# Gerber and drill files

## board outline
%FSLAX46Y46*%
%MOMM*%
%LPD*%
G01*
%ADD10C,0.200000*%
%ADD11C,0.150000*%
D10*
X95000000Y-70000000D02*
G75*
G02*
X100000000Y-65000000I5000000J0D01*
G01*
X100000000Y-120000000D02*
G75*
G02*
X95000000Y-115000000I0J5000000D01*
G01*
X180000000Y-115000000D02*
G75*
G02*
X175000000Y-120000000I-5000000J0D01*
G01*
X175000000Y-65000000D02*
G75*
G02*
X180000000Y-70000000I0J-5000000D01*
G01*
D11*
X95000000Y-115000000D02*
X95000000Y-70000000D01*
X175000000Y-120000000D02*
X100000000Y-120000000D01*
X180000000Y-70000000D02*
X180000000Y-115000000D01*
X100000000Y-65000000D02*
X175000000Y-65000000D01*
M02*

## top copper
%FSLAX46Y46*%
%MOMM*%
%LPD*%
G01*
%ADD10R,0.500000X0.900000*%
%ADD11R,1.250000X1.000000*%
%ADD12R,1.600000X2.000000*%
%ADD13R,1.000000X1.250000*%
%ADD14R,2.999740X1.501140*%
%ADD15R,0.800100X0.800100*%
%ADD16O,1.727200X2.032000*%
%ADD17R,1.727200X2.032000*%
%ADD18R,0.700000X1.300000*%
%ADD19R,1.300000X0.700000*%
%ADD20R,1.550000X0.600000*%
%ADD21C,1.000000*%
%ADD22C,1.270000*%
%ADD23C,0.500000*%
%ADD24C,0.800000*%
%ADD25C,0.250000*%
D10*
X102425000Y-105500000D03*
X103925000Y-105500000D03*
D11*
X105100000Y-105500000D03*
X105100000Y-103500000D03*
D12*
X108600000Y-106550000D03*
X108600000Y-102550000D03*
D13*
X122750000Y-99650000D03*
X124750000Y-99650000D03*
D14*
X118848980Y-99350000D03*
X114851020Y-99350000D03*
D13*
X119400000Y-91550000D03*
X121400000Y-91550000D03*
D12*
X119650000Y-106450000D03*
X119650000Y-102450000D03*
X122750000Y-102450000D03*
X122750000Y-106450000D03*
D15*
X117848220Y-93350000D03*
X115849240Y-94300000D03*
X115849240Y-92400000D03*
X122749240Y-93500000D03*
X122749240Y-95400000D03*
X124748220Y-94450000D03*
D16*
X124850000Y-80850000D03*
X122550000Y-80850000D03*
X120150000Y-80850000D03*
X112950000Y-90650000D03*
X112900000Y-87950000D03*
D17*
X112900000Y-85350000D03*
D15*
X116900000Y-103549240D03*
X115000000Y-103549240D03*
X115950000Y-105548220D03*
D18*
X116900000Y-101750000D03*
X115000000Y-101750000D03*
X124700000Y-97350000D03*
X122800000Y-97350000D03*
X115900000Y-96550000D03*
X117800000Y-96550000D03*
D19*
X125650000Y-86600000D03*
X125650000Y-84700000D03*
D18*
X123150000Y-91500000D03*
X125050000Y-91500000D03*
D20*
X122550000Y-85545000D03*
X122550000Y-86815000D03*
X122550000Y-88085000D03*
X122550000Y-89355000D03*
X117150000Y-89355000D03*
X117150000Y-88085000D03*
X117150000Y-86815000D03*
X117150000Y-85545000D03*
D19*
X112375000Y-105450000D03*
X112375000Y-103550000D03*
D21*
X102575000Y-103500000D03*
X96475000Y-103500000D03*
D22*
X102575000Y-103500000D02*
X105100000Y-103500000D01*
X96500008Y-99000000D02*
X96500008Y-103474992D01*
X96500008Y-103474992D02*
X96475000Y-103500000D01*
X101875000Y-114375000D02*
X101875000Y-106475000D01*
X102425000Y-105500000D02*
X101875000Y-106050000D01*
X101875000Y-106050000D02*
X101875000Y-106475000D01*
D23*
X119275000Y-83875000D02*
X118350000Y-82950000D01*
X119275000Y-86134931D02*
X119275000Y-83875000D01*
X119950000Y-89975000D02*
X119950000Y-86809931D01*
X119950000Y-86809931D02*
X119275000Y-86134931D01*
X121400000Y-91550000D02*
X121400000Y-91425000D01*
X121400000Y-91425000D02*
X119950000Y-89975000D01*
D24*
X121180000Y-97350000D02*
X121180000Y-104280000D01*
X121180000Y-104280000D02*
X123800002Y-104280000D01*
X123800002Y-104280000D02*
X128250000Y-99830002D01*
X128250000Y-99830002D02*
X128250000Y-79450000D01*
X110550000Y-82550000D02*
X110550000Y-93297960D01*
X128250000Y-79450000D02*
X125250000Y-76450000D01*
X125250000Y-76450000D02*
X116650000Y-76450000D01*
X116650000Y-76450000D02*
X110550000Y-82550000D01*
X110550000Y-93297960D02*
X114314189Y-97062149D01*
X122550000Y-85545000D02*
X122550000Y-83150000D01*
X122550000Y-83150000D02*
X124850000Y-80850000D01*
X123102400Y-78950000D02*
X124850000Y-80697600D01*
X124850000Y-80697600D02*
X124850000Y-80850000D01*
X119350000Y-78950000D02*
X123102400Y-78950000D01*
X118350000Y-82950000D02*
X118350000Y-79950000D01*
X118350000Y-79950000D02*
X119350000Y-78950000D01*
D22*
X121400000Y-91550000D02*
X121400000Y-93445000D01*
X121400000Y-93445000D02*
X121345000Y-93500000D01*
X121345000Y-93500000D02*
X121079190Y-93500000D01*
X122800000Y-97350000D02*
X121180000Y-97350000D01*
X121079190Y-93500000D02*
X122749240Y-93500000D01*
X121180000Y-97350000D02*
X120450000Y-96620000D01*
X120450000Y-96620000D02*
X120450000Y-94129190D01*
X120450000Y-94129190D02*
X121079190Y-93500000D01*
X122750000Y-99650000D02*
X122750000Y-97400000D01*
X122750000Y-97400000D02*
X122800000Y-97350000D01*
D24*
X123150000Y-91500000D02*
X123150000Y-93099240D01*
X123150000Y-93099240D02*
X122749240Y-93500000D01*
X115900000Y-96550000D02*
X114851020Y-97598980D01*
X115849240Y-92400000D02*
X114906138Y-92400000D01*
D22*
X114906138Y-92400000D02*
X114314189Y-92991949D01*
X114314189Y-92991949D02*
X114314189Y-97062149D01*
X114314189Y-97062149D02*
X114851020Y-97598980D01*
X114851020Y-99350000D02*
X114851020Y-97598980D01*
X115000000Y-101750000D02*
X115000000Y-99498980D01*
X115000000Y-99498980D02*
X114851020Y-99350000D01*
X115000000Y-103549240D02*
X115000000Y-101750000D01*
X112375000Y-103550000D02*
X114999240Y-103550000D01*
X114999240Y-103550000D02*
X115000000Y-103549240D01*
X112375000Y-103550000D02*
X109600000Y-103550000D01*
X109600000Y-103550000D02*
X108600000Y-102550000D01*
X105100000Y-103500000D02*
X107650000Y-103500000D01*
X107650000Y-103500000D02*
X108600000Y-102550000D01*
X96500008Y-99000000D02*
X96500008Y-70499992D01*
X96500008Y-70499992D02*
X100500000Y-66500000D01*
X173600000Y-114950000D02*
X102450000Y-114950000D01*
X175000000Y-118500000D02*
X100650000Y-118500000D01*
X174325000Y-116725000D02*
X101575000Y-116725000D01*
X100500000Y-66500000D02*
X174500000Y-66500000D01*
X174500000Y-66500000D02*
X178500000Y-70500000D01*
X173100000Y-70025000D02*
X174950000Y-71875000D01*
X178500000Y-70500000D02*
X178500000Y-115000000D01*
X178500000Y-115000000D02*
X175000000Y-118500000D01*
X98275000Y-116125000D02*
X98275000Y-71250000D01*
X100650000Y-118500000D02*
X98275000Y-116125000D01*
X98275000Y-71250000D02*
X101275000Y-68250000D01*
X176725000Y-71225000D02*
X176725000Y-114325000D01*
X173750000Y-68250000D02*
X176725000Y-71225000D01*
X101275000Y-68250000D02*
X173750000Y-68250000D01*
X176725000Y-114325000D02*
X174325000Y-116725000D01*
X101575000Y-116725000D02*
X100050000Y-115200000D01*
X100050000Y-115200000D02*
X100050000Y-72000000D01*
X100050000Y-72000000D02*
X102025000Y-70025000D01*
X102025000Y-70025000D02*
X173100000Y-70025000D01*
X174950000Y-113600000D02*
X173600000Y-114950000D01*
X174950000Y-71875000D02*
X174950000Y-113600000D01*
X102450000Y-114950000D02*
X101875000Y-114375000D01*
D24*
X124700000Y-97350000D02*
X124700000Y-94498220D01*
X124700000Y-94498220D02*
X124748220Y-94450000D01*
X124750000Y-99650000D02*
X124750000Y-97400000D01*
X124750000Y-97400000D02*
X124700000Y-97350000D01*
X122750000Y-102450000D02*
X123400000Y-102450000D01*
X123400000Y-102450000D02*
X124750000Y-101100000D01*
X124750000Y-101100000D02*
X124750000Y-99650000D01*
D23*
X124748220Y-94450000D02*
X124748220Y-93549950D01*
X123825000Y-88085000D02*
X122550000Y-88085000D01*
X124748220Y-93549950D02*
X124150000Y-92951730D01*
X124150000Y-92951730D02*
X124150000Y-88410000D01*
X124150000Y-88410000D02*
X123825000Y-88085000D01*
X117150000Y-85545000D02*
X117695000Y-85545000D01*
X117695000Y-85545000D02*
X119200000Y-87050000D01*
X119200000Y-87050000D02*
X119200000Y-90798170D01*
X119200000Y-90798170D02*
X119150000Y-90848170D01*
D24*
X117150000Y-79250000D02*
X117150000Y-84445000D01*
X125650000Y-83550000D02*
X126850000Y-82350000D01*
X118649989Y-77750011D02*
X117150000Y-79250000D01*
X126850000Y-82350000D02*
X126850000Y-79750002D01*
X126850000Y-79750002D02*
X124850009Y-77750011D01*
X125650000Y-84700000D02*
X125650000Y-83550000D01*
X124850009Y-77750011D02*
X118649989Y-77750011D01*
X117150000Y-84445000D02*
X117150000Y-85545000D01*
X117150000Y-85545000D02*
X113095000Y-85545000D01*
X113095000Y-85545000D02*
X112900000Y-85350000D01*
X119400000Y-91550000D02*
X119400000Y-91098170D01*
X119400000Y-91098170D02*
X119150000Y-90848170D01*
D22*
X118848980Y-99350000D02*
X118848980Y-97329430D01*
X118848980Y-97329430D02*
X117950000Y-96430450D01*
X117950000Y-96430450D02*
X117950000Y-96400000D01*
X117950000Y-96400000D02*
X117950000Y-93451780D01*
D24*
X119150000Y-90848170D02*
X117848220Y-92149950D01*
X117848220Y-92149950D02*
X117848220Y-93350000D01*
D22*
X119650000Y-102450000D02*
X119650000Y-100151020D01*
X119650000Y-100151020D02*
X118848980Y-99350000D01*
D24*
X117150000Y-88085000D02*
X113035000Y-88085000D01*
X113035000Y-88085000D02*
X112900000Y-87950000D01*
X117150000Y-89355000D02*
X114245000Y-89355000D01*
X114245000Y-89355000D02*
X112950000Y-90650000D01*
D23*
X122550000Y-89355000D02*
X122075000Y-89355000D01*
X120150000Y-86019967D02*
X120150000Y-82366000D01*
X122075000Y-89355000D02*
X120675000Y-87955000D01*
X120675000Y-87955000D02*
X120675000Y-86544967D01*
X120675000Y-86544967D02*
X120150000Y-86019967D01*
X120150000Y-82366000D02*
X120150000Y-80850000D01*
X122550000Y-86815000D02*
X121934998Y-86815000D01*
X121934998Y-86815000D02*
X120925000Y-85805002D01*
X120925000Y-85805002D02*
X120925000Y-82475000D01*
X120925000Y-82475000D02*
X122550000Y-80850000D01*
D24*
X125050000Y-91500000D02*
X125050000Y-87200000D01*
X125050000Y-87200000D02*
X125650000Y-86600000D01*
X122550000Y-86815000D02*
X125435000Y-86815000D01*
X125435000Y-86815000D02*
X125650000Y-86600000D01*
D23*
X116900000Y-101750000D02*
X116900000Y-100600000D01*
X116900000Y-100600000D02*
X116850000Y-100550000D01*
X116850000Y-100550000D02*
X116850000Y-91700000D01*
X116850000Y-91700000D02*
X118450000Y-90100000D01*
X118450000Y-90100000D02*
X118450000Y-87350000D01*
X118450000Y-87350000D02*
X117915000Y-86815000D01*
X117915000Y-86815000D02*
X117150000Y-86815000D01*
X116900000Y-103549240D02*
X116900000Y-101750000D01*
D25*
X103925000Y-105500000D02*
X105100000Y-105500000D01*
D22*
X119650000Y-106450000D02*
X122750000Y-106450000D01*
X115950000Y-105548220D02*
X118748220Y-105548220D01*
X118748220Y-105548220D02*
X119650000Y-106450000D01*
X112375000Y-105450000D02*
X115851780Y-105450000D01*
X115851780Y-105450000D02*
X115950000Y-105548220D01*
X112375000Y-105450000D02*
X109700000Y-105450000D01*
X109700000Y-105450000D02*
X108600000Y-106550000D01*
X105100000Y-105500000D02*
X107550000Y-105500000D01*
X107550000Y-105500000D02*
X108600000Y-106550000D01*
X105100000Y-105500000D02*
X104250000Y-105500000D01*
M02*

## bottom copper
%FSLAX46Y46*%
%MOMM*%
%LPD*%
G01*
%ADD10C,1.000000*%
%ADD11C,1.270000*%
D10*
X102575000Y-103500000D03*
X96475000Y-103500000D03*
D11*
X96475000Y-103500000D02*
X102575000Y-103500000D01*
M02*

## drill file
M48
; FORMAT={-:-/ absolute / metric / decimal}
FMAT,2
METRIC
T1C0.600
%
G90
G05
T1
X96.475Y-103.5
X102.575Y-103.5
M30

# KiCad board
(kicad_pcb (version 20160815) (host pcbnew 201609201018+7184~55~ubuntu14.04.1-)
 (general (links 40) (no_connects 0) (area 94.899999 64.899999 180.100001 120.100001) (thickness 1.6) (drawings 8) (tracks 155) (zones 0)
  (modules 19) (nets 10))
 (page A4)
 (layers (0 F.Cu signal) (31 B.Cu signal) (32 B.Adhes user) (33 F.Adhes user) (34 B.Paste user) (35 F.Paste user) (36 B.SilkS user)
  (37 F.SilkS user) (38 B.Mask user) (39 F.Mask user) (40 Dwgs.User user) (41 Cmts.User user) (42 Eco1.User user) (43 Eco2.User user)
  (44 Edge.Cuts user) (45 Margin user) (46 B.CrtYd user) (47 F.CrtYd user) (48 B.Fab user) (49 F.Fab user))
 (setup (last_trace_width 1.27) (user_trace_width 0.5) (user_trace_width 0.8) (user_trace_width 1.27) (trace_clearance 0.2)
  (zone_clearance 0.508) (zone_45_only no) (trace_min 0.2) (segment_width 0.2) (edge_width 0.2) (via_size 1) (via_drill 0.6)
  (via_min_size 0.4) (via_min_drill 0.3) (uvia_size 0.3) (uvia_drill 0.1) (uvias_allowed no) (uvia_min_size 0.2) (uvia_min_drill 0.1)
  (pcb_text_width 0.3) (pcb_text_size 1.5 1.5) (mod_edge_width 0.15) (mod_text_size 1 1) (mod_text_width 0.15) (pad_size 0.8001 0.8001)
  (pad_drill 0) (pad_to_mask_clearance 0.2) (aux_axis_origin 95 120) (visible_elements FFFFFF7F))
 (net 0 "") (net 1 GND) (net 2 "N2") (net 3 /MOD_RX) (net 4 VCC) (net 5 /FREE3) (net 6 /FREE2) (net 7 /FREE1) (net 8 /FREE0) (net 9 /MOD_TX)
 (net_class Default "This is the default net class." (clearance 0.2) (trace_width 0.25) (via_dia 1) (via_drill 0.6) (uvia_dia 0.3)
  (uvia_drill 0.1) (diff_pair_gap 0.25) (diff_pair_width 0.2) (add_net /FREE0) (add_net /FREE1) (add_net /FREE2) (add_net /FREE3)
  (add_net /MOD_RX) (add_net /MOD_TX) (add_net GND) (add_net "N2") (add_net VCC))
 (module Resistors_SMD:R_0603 (layer F.Cu) (at 103.175 105.5 180)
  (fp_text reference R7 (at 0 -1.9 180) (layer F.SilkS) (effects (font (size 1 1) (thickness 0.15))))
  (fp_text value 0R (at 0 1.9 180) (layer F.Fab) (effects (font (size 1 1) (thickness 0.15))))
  (pad 2 smd rect (at 0.75 0 180) (size 0.5 0.9) (layers F.Cu F.Paste F.Mask) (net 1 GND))
  (pad 1 smd rect (at -0.75 0 180) (size 0.5 0.9) (layers F.Cu F.Paste F.Mask) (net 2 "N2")))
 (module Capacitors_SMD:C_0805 (layer F.Cu) (at 105.1 104.5 90)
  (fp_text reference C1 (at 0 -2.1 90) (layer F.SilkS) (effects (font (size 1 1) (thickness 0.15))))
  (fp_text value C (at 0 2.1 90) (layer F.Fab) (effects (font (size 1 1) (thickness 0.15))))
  (pad 1 smd rect (at -1 0 90) (size 1 1.25) (layers F.Cu F.Paste F.Mask) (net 2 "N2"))
  (pad 2 smd rect (at 1 0 90) (size 1 1.25) (layers F.Cu F.Paste F.Mask) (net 1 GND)))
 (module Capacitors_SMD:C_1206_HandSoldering (layer F.Cu) (at 108.6 104.55 90)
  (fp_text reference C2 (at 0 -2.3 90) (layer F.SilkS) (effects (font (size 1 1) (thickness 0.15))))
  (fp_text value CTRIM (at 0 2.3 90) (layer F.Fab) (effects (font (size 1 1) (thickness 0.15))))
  (pad 1 smd rect (at -2 0 90) (size 2 1.6) (layers F.Cu F.Paste F.Mask) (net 2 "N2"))
  (pad 2 smd rect (at 2 0 90) (size 2 1.6) (layers F.Cu F.Paste F.Mask) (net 1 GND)))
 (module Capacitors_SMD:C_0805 (layer F.Cu) (at 123.75 99.65 180)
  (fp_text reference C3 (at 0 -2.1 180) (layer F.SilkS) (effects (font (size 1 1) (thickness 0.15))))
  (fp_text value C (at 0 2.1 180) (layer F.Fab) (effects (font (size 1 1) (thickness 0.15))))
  (pad 2 smd rect (at 1 0 180) (size 1 1.25) (layers F.Cu F.Paste F.Mask) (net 1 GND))
  (pad 1 smd rect (at -1 0 180) (size 1 1.25) (layers F.Cu F.Paste F.Mask) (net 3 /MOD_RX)))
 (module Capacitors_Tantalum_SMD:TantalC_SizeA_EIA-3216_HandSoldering (layer F.Cu) (at 116.85 99.35 180)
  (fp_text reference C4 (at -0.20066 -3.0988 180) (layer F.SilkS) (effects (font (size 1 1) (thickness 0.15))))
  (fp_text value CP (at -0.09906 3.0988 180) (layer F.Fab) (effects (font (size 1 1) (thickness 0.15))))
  (pad 1 smd rect (at -1.99898 0 180) (size 2.99974 1.50114) (layers F.Cu F.Paste F.Mask) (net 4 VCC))
  (pad 2 smd rect (at 1.99898 0 180) (size 2.99974 1.50114) (layers F.Cu F.Paste F.Mask) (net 1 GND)))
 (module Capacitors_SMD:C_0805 (layer F.Cu) (at 120.4 91.55)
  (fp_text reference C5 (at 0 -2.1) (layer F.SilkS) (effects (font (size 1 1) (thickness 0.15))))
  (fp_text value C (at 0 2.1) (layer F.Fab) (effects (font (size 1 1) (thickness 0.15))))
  (pad 1 smd rect (at -1 0) (size 1 1.25) (layers F.Cu F.Paste F.Mask) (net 4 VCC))
  (pad 2 smd rect (at 1 0) (size 1 1.25) (layers F.Cu F.Paste F.Mask) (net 1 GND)))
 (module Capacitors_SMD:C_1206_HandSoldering (layer F.Cu) (at 119.65 104.45 270)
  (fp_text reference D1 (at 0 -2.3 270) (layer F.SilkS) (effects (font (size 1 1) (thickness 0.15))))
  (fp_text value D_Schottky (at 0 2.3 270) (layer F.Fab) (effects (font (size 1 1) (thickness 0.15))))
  (pad 2 smd rect (at 2 0 270) (size 2 1.6) (layers F.Cu F.Paste F.Mask) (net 2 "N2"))
  (pad 1 smd rect (at -2 0 270) (size 2 1.6) (layers F.Cu F.Paste F.Mask) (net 4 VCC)))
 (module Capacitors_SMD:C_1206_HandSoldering (layer F.Cu) (at 122.75 104.45 270)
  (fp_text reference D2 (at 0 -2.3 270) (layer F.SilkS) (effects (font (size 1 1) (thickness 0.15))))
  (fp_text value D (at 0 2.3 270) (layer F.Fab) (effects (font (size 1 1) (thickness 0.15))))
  (pad 1 smd rect (at -2 0 270) (size 2 1.6) (layers F.Cu F.Paste F.Mask) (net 3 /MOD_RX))
  (pad 2 smd rect (at 2 0 270) (size 2 1.6) (layers F.Cu F.Paste F.Mask) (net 2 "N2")))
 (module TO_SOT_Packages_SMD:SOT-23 (layer F.Cu) (at 116.85 93.35 270)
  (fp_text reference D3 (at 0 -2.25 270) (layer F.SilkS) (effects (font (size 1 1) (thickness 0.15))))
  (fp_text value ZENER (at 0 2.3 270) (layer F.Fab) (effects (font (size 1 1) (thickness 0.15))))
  (pad 1 smd rect (at 0 -0.99822 270) (size 0.8001 0.8001) (layers F.Cu F.Paste F.Mask) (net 4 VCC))
  (pad 3 smd rect (at 0.95 1.00076 270) (size 0.8001 0.8001) (layers F.Cu F.Paste F.Mask))
  (pad 2 smd rect (at -0.95 1.00076 270) (size 0.8001 0.8001) (layers F.Cu F.Paste F.Mask) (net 1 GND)))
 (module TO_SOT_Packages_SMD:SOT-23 (layer F.Cu) (at 123.75 94.45 270)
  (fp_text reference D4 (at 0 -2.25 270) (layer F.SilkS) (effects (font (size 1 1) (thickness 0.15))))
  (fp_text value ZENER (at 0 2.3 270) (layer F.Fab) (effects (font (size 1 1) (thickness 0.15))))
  (pad 2 smd rect (at -0.95 1.00076 270) (size 0.8001 0.8001) (layers F.Cu F.Paste F.Mask) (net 1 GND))
  (pad 3 smd rect (at 0.95 1.00076 270) (size 0.8001 0.8001) (layers F.Cu F.Paste F.Mask))
  (pad 1 smd rect (at 0 -0.99822 270) (size 0.8001 0.8001) (layers F.Cu F.Paste F.Mask) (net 3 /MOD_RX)))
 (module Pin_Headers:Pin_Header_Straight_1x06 (layer F.Cu) (at 114.17 80.65 90)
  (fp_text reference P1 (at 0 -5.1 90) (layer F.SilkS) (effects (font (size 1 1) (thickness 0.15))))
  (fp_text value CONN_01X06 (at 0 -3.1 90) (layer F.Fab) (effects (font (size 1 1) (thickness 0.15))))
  (pad 6 smd oval (at -0.2 10.68 90) (size 2.032 1.7272) (layers F.Cu F.Paste F.Mask) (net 1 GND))
  (pad 5 smd oval (at -0.2 8.38 90) (size 2.032 1.7272) (layers F.Cu F.Paste F.Mask) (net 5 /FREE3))
  (pad 4 smd oval (at -0.2 5.98 90) (size 2.032 1.7272) (layers F.Cu F.Paste F.Mask) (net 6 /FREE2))
  (pad 3 smd oval (at -10 -1.22 90) (size 2.032 1.7272) (layers F.Cu F.Paste F.Mask) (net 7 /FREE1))
  (pad 2 smd oval (at -7.3 -1.27 90) (size 2.032 1.7272) (layers F.Cu F.Paste F.Mask) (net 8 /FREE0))
  (pad 1 smd rect (at -4.7 -1.27 90) (size 2.032 1.7272) (layers F.Cu F.Paste F.Mask) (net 4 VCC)))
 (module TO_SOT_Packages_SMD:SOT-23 (layer F.Cu) (at 115.95 104.55 180)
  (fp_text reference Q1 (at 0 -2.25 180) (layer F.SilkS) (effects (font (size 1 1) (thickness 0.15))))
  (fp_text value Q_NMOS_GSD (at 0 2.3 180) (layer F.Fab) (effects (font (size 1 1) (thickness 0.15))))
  (pad 1 smd rect (at -0.95 1.00076 180) (size 0.8001 0.8001) (layers F.Cu F.Paste F.Mask) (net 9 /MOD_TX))
  (pad 2 smd rect (at 0.95 1.00076 180) (size 0.8001 0.8001) (layers F.Cu F.Paste F.Mask) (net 1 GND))
  (pad 3 smd rect (at 0 -0.99822 180) (size 0.8001 0.8001) (layers F.Cu F.Paste F.Mask) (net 2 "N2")))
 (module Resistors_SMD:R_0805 (layer F.Cu) (at 115.95 101.75 180)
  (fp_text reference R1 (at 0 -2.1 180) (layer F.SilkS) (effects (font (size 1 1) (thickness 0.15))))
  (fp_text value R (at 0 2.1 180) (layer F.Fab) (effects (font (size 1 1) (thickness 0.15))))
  (pad 1 smd rect (at -0.95 0 180) (size 0.7 1.3) (layers F.Cu F.Paste F.Mask) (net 9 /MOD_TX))
  (pad 2 smd rect (at 0.95 0 180) (size 0.7 1.3) (layers F.Cu F.Paste F.Mask) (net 1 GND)))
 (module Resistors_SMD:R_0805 (layer F.Cu) (at 123.75 97.35 180)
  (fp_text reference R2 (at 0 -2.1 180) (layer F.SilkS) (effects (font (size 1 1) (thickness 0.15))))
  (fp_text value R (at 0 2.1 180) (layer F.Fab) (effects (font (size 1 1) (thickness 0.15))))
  (pad 1 smd rect (at -0.95 0 180) (size 0.7 1.3) (layers F.Cu F.Paste F.Mask) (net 3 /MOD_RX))
  (pad 2 smd rect (at 0.95 0 180) (size 0.7 1.3) (layers F.Cu F.Paste F.Mask) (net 1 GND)))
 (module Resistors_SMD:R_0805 (layer F.Cu) (at 116.85 96.55 180)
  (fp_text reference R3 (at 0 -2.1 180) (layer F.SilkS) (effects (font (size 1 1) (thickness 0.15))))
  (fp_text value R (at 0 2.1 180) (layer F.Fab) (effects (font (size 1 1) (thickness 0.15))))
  (pad 2 smd rect (at 0.95 0 180) (size 0.7 1.3) (layers F.Cu F.Paste F.Mask) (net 1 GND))
  (pad 1 smd rect (at -0.95 0 180) (size 0.7 1.3) (layers F.Cu F.Paste F.Mask) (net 4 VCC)))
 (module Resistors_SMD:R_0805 (layer F.Cu) (at 125.65 85.65 270)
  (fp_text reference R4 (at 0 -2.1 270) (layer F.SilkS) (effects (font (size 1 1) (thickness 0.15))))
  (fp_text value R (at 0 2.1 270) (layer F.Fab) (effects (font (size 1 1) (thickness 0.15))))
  (pad 2 smd rect (at 0.95 0 270) (size 0.7 1.3) (layers F.Cu F.Paste F.Mask) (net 5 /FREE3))
  (pad 1 smd rect (at -0.95 0 270) (size 0.7 1.3) (layers F.Cu F.Paste F.Mask) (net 4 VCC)))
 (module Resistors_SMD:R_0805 (layer F.Cu) (at 124.1 91.5 180)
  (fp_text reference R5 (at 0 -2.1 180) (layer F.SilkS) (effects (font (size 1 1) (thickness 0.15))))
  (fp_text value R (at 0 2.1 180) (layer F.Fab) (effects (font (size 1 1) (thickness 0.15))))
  (pad 2 smd rect (at 0.95 0 180) (size 0.7 1.3) (layers F.Cu F.Paste F.Mask) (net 1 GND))
  (pad 1 smd rect (at -0.95 0 180) (size 0.7 1.3) (layers F.Cu F.Paste F.Mask) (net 5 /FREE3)))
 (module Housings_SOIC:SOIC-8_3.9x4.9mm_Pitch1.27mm (layer F.Cu) (at 119.85 87.45)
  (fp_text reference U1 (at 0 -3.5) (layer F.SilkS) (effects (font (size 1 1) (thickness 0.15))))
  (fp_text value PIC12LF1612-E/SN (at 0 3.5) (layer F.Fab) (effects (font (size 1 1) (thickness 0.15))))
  (pad 8 smd rect (at 2.7 -1.905) (size 1.55 0.6) (layers F.Cu F.Paste F.Mask) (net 1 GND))
  (pad 7 smd rect (at 2.7 -0.635) (size 1.55 0.6) (layers F.Cu F.Paste F.Mask) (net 5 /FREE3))
  (pad 6 smd rect (at 2.7 0.635) (size 1.55 0.6) (layers F.Cu F.Paste F.Mask) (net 3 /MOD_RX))
  (pad 5 smd rect (at 2.7 1.905) (size 1.55 0.6) (layers F.Cu F.Paste F.Mask) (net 6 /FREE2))
  (pad 4 smd rect (at -2.7 1.905) (size 1.55 0.6) (layers F.Cu F.Paste F.Mask) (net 7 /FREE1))
  (pad 3 smd rect (at -2.7 0.635) (size 1.55 0.6) (layers F.Cu F.Paste F.Mask) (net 8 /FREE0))
  (pad 2 smd rect (at -2.7 -0.635) (size 1.55 0.6) (layers F.Cu F.Paste F.Mask) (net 9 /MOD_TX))
  (pad 1 smd rect (at -2.7 -1.905) (size 1.55 0.6) (layers F.Cu F.Paste F.Mask) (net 4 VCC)))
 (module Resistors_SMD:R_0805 (layer F.Cu) (at 112.375 104.5 90)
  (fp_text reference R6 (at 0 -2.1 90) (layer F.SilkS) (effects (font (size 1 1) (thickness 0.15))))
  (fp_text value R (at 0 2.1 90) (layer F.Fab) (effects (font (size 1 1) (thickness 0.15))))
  (pad 1 smd rect (at -0.95 0 90) (size 0.7 1.3) (layers F.Cu F.Paste F.Mask) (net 2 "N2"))
  (pad 2 smd rect (at 0.95 0 90) (size 0.7 1.3) (layers F.Cu F.Paste F.Mask) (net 1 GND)))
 (gr_arc (start 100 70) (end 95 70) (angle 90) (layer Edge.Cuts) (width 0.2))
 (gr_arc (start 100 115) (end 100 120) (angle 90) (layer Edge.Cuts) (width 0.2))
 (gr_arc (start 175 115) (end 180 115) (angle 90) (layer Edge.Cuts) (width 0.2))
 (gr_arc (start 175 70) (end 175 65) (angle 90) (layer Edge.Cuts) (width 0.2))
 (gr_line (start 95 115) (end 95 70) (layer Edge.Cuts) (width 0.15))
 (gr_line (start 175 120) (end 100 120) (layer Edge.Cuts) (width 0.15))
 (gr_line (start 180 70) (end 180 115) (layer Edge.Cuts) (width 0.15))
 (gr_line (start 100 65) (end 175 65) (layer Edge.Cuts) (width 0.15))
 (segment (start 102.575 103.5) (end 105.1 103.5) (width 1.27) (layer F.Cu) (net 1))
 (segment (start 96.475 103.5) (end 102.575 103.5) (width 1.27) (layer B.Cu) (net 1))
 (via (at 102.575 103.5) (size 1) (drill 0.6) (layers F.Cu B.Cu) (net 1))
 (segment (start 96.500008 99) (end 96.500008 103.474992) (width 1.27) (layer F.Cu) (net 1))
 (segment (start 96.500008 103.474992) (end 96.475 103.5) (width 1.27) (layer F.Cu) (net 1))
 (via (at 96.475 103.5) (size 1) (drill 0.6) (layers F.Cu B.Cu) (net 1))
 (segment (start 101.875 114.375) (end 101.875 106.475) (width 1.27) (layer F.Cu) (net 1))
 (segment (start 102.425 105.5) (end 101.875 106.05) (width 1.27) (layer F.Cu) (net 1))
 (segment (start 101.875 106.05) (end 101.875 106.475) (width 1.27) (layer F.Cu) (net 1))
 (segment (start 119.275 83.875) (end 118.35 82.95) (width 0.5) (layer F.Cu) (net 1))
 (segment (start 119.275 86.134931) (end 119.275 83.875) (width 0.5) (layer F.Cu) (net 1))
 (segment (start 119.95 89.975) (end 119.95 86.809931) (width 0.5) (layer F.Cu) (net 1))
 (segment (start 119.95 86.809931) (end 119.275 86.134931) (width 0.5) (layer F.Cu) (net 1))
 (segment (start 121.4 91.55) (end 121.4 91.425) (width 0.5) (layer F.Cu) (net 1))
 (segment (start 121.4 91.425) (end 119.95 89.975) (width 0.5) (layer F.Cu) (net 1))
 (segment (start 121.18 97.35) (end 121.18 104.28) (width 0.8) (layer F.Cu) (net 1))
 (segment (start 121.18 104.28) (end 123.800002 104.28) (width 0.8) (layer F.Cu) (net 1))
 (segment (start 123.800002 104.28) (end 128.25 99.830002) (width 0.8) (layer F.Cu) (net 1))
 (segment (start 128.25 99.830002) (end 128.25 79.45) (width 0.8) (layer F.Cu) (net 1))
 (segment (start 110.55 82.55) (end 110.55 93.29796) (width 0.8) (layer F.Cu) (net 1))
 (segment (start 128.25 79.45) (end 125.25 76.45) (width 0.8) (layer F.Cu) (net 1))
 (segment (start 125.25 76.45) (end 116.65 76.45) (width 0.8) (layer F.Cu) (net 1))
 (segment (start 116.65 76.45) (end 110.55 82.55) (width 0.8) (layer F.Cu) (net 1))
 (segment (start 110.55 93.29796) (end 114.314189 97.062149) (width 0.8) (layer F.Cu) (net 1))
 (segment (start 122.55 85.545) (end 122.55 83.15) (width 0.8) (layer F.Cu) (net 1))
 (segment (start 122.55 83.15) (end 124.85 80.85) (width 0.8) (layer F.Cu) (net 1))
 (segment (start 123.1024 78.95) (end 124.85 80.6976) (width 0.8) (layer F.Cu) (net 1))
 (segment (start 124.85 80.6976) (end 124.85 80.85) (width 0.8) (layer F.Cu) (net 1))
 (segment (start 119.35 78.95) (end 123.1024 78.95) (width 0.8) (layer F.Cu) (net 1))
 (segment (start 118.35 82.95) (end 118.35 79.95) (width 0.8) (layer F.Cu) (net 1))
 (segment (start 118.35 79.95) (end 119.35 78.95) (width 0.8) (layer F.Cu) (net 1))
 (segment (start 121.4 91.55) (end 121.4 93.445) (width 1.27) (layer F.Cu) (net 1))
 (segment (start 121.4 93.445) (end 121.345 93.5) (width 1.27) (layer F.Cu) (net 1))
 (segment (start 121.345 93.5) (end 121.07919 93.5) (width 1.27) (layer F.Cu) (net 1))
 (segment (start 122.8 97.35) (end 121.18 97.35) (width 1.27) (layer F.Cu) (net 1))
 (segment (start 121.07919 93.5) (end 122.74924 93.5) (width 1.27) (layer F.Cu) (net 1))
 (segment (start 121.18 97.35) (end 120.45 96.62) (width 1.27) (layer F.Cu) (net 1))
 (segment (start 120.45 96.62) (end 120.45 94.12919) (width 1.27) (layer F.Cu) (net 1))
 (segment (start 120.45 94.12919) (end 121.07919 93.5) (width 1.27) (layer F.Cu) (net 1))
 (segment (start 122.75 99.65) (end 122.75 97.4) (width 1.27) (layer F.Cu) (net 1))
 (segment (start 122.75 97.4) (end 122.8 97.35) (width 1.27) (layer F.Cu) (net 1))
 (segment (start 123.15 91.5) (end 123.15 93.09924) (width 0.8) (layer F.Cu) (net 1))
 (segment (start 123.15 93.09924) (end 122.74924 93.5) (width 0.8) (layer F.Cu) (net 1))
 (segment (start 115.9 96.55) (end 114.85102 97.59898) (width 0.8) (layer F.Cu) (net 1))
 (segment (start 115.84924 92.4) (end 114.906138 92.4) (width 0.8) (layer F.Cu) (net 1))
 (segment (start 114.906138 92.4) (end 114.314189 92.991949) (width 1.27) (layer F.Cu) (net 1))
 (segment (start 114.314189 92.991949) (end 114.314189 97.062149) (width 1.27) (layer F.Cu) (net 1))
 (segment (start 114.314189 97.062149) (end 114.85102 97.59898) (width 1.27) (layer F.Cu) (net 1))
 (segment (start 114.85102 99.35) (end 114.85102 97.59898) (width 1.27) (layer F.Cu) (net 1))
 (segment (start 115 101.75) (end 115 99.49898) (width 1.27) (layer F.Cu) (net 1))
 (segment (start 115 99.49898) (end 114.85102 99.35) (width 1.27) (layer F.Cu) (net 1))
 (segment (start 115 103.54924) (end 115 101.75) (width 1.27) (layer F.Cu) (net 1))
 (segment (start 112.375 103.55) (end 114.99924 103.55) (width 1.27) (layer F.Cu) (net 1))
 (segment (start 114.99924 103.55) (end 115 103.54924) (width 1.27) (layer F.Cu) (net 1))
 (segment (start 112.375 103.55) (end 109.6 103.55) (width 1.27) (layer F.Cu) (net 1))
 (segment (start 109.6 103.55) (end 108.6 102.55) (width 1.27) (layer F.Cu) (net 1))
 (segment (start 105.1 103.5) (end 107.65 103.5) (width 1.27) (layer F.Cu) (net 1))
 (segment (start 107.65 103.5) (end 108.6 102.55) (width 1.27) (layer F.Cu) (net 1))
 (segment (start 96.500008 99) (end 96.500008 70.499992) (width 1.27) (layer F.Cu) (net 1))
 (segment (start 96.500008 70.499992) (end 100.5 66.5) (width 1.27) (layer F.Cu) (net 1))
 (segment (start 173.6 114.95) (end 102.45 114.95) (width 1.27) (layer F.Cu) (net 1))
 (segment (start 175 118.5) (end 100.65 118.5) (width 1.27) (layer F.Cu) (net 1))
 (segment (start 174.325 116.725) (end 101.575 116.725) (width 1.27) (layer F.Cu) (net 1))
 (segment (start 100.5 66.5) (end 174.5 66.5) (width 1.27) (layer F.Cu) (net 1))
 (segment (start 174.5 66.5) (end 178.5 70.5) (width 1.27) (layer F.Cu) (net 1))
 (segment (start 173.1 70.025) (end 174.95 71.875) (width 1.27) (layer F.Cu) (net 1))
 (segment (start 178.5 70.5) (end 178.5 115) (width 1.27) (layer F.Cu) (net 1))
 (segment (start 178.5 115) (end 175 118.5) (width 1.27) (layer F.Cu) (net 1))
 (segment (start 98.275 116.125) (end 98.275 71.25) (width 1.27) (layer F.Cu) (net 1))
 (segment (start 100.65 118.5) (end 98.275 116.125) (width 1.27) (layer F.Cu) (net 1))
 (segment (start 98.275 71.25) (end 101.275 68.25) (width 1.27) (layer F.Cu) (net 1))
 (segment (start 176.725 71.225) (end 176.725 114.325) (width 1.27) (layer F.Cu) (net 1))
 (segment (start 173.75 68.25) (end 176.725 71.225) (width 1.27) (layer F.Cu) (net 1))
 (segment (start 101.275 68.25) (end 173.75 68.25) (width 1.27) (layer F.Cu) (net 1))
 (segment (start 176.725 114.325) (end 174.325 116.725) (width 1.27) (layer F.Cu) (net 1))
 (segment (start 101.575 116.725) (end 100.05 115.2) (width 1.27) (layer F.Cu) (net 1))
 (segment (start 100.05 115.2) (end 100.05 72) (width 1.27) (layer F.Cu) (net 1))
 (segment (start 100.05 72) (end 102.025 70.025) (width 1.27) (layer F.Cu) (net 1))
 (segment (start 102.025 70.025) (end 173.1 70.025) (width 1.27) (layer F.Cu) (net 1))
 (segment (start 174.95 113.6) (end 173.6 114.95) (width 1.27) (layer F.Cu) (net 1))
 (segment (start 174.95 71.875) (end 174.95 113.6) (width 1.27) (layer F.Cu) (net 1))
 (segment (start 102.45 114.95) (end 101.875 114.375) (width 1.27) (layer F.Cu) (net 1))
 (segment (start 124.7 97.35) (end 124.7 94.49822) (width 0.8) (layer F.Cu) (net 3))
 (segment (start 124.7 94.49822) (end 124.74822 94.45) (width 0.8) (layer F.Cu) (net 3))
 (segment (start 124.75 99.65) (end 124.75 97.4) (width 0.8) (layer F.Cu) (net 3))
 (segment (start 124.75 97.4) (end 124.7 97.35) (width 0.8) (layer F.Cu) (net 3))
 (segment (start 122.75 102.45) (end 123.4 102.45) (width 0.8) (layer F.Cu) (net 3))
 (segment (start 123.4 102.45) (end 124.75 101.1) (width 0.8) (layer F.Cu) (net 3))
 (segment (start 124.75 101.1) (end 124.75 99.65) (width 0.8) (layer F.Cu) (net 3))
 (segment (start 124.74822 94.45) (end 124.74822 93.54995) (width 0.5) (layer F.Cu) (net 3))
 (segment (start 123.825 88.085) (end 122.55 88.085) (width 0.5) (layer F.Cu) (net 3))
 (segment (start 124.74822 93.54995) (end 124.15 92.95173) (width 0.5) (layer F.Cu) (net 3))
 (segment (start 124.15 92.95173) (end 124.15 88.41) (width 0.5) (layer F.Cu) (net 3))
 (segment (start 124.15 88.41) (end 123.825 88.085) (width 0.5) (layer F.Cu) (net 3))
 (segment (start 117.15 85.545) (end 117.695 85.545) (width 0.5) (layer F.Cu) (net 4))
 (segment (start 117.695 85.545) (end 119.2 87.05) (width 0.5) (layer F.Cu) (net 4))
 (segment (start 119.2 87.05) (end 119.2 90.79817) (width 0.5) (layer F.Cu) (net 4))
 (segment (start 119.2 90.79817) (end 119.15 90.84817) (width 0.5) (layer F.Cu) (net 4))
 (segment (start 117.15 79.25) (end 117.15 84.445) (width 0.8) (layer F.Cu) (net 4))
 (segment (start 125.65 83.55) (end 126.85 82.35) (width 0.8) (layer F.Cu) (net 4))
 (segment (start 118.649989 77.750011) (end 117.15 79.25) (width 0.8) (layer F.Cu) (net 4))
 (segment (start 126.85 82.35) (end 126.85 79.750002) (width 0.8) (layer F.Cu) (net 4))
 (segment (start 126.85 79.750002) (end 124.850009 77.750011) (width 0.8) (layer F.Cu) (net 4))
 (segment (start 125.65 84.7) (end 125.65 83.55) (width 0.8) (layer F.Cu) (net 4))
 (segment (start 124.850009 77.750011) (end 118.649989 77.750011) (width 0.8) (layer F.Cu) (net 4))
 (segment (start 117.15 84.445) (end 117.15 85.545) (width 0.8) (layer F.Cu) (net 4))
 (segment (start 117.15 85.545) (end 113.095 85.545) (width 0.8) (layer F.Cu) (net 4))
 (segment (start 113.095 85.545) (end 112.9 85.35) (width 0.8) (layer F.Cu) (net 4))
 (segment (start 119.4 91.55) (end 119.4 91.09817) (width 0.8) (layer F.Cu) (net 4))
 (segment (start 119.4 91.09817) (end 119.15 90.84817) (width 0.8) (layer F.Cu) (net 4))
 (segment (start 118.84898 99.35) (end 118.84898 97.32943) (width 1.27) (layer F.Cu) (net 4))
 (segment (start 118.84898 97.32943) (end 117.95 96.43045) (width 1.27) (layer F.Cu) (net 4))
 (segment (start 117.95 96.43045) (end 117.95 96.4) (width 1.27) (layer F.Cu) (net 4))
 (segment (start 117.95 96.4) (end 117.95 93.45178) (width 1.27) (layer F.Cu) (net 4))
 (segment (start 119.15 90.84817) (end 117.84822 92.14995) (width 0.8) (layer F.Cu) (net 4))
 (segment (start 117.84822 92.14995) (end 117.84822 93.35) (width 0.8) (layer F.Cu) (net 4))
 (segment (start 119.65 102.45) (end 119.65 100.15102) (width 1.27) (layer F.Cu) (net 4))
 (segment (start 119.65 100.15102) (end 118.84898 99.35) (width 1.27) (layer F.Cu) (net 4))
 (segment (start 117.15 88.085) (end 113.035 88.085) (width 0.8) (layer F.Cu) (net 8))
 (segment (start 113.035 88.085) (end 112.9 87.95) (width 0.8) (layer F.Cu) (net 8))
 (segment (start 117.15 89.355) (end 114.245 89.355) (width 0.8) (layer F.Cu) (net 7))
 (segment (start 114.245 89.355) (end 112.95 90.65) (width 0.8) (layer F.Cu) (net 7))
 (segment (start 122.55 89.355) (end 122.075 89.355) (width 0.5) (layer F.Cu) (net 6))
 (segment (start 120.15 86.019967) (end 120.15 82.366) (width 0.5) (layer F.Cu) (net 6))
 (segment (start 122.075 89.355) (end 120.675 87.955) (width 0.5) (layer F.Cu) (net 6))
 (segment (start 120.675 87.955) (end 120.675 86.544967) (width 0.5) (layer F.Cu) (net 6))
 (segment (start 120.675 86.544967) (end 120.15 86.019967) (width 0.5) (layer F.Cu) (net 6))
 (segment (start 120.15 82.366) (end 120.15 80.85) (width 0.5) (layer F.Cu) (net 6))
 (segment (start 122.55 86.815) (end 121.934998 86.815) (width 0.5) (layer F.Cu) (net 5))
 (segment (start 121.934998 86.815) (end 120.925 85.805002) (width 0.5) (layer F.Cu) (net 5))
 (segment (start 120.925 85.805002) (end 120.925 82.475) (width 0.5) (layer F.Cu) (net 5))
 (segment (start 120.925 82.475) (end 122.55 80.85) (width 0.5) (layer F.Cu) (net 5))
 (segment (start 125.05 91.5) (end 125.05 87.2) (width 0.8) (layer F.Cu) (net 5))
 (segment (start 125.05 87.2) (end 125.65 86.6) (width 0.8) (layer F.Cu) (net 5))
 (segment (start 122.55 86.815) (end 125.435 86.815) (width 0.8) (layer F.Cu) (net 5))
 (segment (start 125.435 86.815) (end 125.65 86.6) (width 0.8) (layer F.Cu) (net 5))
 (segment (start 116.9 101.75) (end 116.9 100.6) (width 0.5) (layer F.Cu) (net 9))
 (segment (start 116.9 100.6) (end 116.85 100.55) (width 0.5) (layer F.Cu) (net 9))
 (segment (start 116.85 100.55) (end 116.85 91.7) (width 0.5) (layer F.Cu) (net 9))
 (segment (start 116.85 91.7) (end 118.45 90.1) (width 0.5) (layer F.Cu) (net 9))
 (segment (start 118.45 90.1) (end 118.45 87.35) (width 0.5) (layer F.Cu) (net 9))
 (segment (start 118.45 87.35) (end 117.915 86.815) (width 0.5) (layer F.Cu) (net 9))
 (segment (start 117.915 86.815) (end 117.15 86.815) (width 0.5) (layer F.Cu) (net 9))
 (segment (start 116.9 103.54924) (end 116.9 101.75) (width 0.5) (layer F.Cu) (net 9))
 (segment (start 103.925 105.5) (end 105.1 105.5) (width 0.25) (layer F.Cu) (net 2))
 (segment (start 119.65 106.45) (end 122.75 106.45) (width 1.27) (layer F.Cu) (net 2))
 (segment (start 115.95 105.54822) (end 118.74822 105.54822) (width 1.27) (layer F.Cu) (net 2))
 (segment (start 118.74822 105.54822) (end 119.65 106.45) (width 1.27) (layer F.Cu) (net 2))
 (segment (start 112.375 105.45) (end 115.85178 105.45) (width 1.27) (layer F.Cu) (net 2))
 (segment (start 115.85178 105.45) (end 115.95 105.54822) (width 1.27) (layer F.Cu) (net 2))
 (segment (start 112.375 105.45) (end 109.7 105.45) (width 1.27) (layer F.Cu) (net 2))
 (segment (start 109.7 105.45) (end 108.6 106.55) (width 1.27) (layer F.Cu) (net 2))
 (segment (start 105.1 105.5) (end 107.55 105.5) (width 1.27) (layer F.Cu) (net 2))
 (segment (start 107.55 105.5) (end 108.6 106.55) (width 1.27) (layer F.Cu) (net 2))
 (segment (start 105.1 105.5) (end 104.25 105.5) (width 1.27) (layer F.Cu) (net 2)))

